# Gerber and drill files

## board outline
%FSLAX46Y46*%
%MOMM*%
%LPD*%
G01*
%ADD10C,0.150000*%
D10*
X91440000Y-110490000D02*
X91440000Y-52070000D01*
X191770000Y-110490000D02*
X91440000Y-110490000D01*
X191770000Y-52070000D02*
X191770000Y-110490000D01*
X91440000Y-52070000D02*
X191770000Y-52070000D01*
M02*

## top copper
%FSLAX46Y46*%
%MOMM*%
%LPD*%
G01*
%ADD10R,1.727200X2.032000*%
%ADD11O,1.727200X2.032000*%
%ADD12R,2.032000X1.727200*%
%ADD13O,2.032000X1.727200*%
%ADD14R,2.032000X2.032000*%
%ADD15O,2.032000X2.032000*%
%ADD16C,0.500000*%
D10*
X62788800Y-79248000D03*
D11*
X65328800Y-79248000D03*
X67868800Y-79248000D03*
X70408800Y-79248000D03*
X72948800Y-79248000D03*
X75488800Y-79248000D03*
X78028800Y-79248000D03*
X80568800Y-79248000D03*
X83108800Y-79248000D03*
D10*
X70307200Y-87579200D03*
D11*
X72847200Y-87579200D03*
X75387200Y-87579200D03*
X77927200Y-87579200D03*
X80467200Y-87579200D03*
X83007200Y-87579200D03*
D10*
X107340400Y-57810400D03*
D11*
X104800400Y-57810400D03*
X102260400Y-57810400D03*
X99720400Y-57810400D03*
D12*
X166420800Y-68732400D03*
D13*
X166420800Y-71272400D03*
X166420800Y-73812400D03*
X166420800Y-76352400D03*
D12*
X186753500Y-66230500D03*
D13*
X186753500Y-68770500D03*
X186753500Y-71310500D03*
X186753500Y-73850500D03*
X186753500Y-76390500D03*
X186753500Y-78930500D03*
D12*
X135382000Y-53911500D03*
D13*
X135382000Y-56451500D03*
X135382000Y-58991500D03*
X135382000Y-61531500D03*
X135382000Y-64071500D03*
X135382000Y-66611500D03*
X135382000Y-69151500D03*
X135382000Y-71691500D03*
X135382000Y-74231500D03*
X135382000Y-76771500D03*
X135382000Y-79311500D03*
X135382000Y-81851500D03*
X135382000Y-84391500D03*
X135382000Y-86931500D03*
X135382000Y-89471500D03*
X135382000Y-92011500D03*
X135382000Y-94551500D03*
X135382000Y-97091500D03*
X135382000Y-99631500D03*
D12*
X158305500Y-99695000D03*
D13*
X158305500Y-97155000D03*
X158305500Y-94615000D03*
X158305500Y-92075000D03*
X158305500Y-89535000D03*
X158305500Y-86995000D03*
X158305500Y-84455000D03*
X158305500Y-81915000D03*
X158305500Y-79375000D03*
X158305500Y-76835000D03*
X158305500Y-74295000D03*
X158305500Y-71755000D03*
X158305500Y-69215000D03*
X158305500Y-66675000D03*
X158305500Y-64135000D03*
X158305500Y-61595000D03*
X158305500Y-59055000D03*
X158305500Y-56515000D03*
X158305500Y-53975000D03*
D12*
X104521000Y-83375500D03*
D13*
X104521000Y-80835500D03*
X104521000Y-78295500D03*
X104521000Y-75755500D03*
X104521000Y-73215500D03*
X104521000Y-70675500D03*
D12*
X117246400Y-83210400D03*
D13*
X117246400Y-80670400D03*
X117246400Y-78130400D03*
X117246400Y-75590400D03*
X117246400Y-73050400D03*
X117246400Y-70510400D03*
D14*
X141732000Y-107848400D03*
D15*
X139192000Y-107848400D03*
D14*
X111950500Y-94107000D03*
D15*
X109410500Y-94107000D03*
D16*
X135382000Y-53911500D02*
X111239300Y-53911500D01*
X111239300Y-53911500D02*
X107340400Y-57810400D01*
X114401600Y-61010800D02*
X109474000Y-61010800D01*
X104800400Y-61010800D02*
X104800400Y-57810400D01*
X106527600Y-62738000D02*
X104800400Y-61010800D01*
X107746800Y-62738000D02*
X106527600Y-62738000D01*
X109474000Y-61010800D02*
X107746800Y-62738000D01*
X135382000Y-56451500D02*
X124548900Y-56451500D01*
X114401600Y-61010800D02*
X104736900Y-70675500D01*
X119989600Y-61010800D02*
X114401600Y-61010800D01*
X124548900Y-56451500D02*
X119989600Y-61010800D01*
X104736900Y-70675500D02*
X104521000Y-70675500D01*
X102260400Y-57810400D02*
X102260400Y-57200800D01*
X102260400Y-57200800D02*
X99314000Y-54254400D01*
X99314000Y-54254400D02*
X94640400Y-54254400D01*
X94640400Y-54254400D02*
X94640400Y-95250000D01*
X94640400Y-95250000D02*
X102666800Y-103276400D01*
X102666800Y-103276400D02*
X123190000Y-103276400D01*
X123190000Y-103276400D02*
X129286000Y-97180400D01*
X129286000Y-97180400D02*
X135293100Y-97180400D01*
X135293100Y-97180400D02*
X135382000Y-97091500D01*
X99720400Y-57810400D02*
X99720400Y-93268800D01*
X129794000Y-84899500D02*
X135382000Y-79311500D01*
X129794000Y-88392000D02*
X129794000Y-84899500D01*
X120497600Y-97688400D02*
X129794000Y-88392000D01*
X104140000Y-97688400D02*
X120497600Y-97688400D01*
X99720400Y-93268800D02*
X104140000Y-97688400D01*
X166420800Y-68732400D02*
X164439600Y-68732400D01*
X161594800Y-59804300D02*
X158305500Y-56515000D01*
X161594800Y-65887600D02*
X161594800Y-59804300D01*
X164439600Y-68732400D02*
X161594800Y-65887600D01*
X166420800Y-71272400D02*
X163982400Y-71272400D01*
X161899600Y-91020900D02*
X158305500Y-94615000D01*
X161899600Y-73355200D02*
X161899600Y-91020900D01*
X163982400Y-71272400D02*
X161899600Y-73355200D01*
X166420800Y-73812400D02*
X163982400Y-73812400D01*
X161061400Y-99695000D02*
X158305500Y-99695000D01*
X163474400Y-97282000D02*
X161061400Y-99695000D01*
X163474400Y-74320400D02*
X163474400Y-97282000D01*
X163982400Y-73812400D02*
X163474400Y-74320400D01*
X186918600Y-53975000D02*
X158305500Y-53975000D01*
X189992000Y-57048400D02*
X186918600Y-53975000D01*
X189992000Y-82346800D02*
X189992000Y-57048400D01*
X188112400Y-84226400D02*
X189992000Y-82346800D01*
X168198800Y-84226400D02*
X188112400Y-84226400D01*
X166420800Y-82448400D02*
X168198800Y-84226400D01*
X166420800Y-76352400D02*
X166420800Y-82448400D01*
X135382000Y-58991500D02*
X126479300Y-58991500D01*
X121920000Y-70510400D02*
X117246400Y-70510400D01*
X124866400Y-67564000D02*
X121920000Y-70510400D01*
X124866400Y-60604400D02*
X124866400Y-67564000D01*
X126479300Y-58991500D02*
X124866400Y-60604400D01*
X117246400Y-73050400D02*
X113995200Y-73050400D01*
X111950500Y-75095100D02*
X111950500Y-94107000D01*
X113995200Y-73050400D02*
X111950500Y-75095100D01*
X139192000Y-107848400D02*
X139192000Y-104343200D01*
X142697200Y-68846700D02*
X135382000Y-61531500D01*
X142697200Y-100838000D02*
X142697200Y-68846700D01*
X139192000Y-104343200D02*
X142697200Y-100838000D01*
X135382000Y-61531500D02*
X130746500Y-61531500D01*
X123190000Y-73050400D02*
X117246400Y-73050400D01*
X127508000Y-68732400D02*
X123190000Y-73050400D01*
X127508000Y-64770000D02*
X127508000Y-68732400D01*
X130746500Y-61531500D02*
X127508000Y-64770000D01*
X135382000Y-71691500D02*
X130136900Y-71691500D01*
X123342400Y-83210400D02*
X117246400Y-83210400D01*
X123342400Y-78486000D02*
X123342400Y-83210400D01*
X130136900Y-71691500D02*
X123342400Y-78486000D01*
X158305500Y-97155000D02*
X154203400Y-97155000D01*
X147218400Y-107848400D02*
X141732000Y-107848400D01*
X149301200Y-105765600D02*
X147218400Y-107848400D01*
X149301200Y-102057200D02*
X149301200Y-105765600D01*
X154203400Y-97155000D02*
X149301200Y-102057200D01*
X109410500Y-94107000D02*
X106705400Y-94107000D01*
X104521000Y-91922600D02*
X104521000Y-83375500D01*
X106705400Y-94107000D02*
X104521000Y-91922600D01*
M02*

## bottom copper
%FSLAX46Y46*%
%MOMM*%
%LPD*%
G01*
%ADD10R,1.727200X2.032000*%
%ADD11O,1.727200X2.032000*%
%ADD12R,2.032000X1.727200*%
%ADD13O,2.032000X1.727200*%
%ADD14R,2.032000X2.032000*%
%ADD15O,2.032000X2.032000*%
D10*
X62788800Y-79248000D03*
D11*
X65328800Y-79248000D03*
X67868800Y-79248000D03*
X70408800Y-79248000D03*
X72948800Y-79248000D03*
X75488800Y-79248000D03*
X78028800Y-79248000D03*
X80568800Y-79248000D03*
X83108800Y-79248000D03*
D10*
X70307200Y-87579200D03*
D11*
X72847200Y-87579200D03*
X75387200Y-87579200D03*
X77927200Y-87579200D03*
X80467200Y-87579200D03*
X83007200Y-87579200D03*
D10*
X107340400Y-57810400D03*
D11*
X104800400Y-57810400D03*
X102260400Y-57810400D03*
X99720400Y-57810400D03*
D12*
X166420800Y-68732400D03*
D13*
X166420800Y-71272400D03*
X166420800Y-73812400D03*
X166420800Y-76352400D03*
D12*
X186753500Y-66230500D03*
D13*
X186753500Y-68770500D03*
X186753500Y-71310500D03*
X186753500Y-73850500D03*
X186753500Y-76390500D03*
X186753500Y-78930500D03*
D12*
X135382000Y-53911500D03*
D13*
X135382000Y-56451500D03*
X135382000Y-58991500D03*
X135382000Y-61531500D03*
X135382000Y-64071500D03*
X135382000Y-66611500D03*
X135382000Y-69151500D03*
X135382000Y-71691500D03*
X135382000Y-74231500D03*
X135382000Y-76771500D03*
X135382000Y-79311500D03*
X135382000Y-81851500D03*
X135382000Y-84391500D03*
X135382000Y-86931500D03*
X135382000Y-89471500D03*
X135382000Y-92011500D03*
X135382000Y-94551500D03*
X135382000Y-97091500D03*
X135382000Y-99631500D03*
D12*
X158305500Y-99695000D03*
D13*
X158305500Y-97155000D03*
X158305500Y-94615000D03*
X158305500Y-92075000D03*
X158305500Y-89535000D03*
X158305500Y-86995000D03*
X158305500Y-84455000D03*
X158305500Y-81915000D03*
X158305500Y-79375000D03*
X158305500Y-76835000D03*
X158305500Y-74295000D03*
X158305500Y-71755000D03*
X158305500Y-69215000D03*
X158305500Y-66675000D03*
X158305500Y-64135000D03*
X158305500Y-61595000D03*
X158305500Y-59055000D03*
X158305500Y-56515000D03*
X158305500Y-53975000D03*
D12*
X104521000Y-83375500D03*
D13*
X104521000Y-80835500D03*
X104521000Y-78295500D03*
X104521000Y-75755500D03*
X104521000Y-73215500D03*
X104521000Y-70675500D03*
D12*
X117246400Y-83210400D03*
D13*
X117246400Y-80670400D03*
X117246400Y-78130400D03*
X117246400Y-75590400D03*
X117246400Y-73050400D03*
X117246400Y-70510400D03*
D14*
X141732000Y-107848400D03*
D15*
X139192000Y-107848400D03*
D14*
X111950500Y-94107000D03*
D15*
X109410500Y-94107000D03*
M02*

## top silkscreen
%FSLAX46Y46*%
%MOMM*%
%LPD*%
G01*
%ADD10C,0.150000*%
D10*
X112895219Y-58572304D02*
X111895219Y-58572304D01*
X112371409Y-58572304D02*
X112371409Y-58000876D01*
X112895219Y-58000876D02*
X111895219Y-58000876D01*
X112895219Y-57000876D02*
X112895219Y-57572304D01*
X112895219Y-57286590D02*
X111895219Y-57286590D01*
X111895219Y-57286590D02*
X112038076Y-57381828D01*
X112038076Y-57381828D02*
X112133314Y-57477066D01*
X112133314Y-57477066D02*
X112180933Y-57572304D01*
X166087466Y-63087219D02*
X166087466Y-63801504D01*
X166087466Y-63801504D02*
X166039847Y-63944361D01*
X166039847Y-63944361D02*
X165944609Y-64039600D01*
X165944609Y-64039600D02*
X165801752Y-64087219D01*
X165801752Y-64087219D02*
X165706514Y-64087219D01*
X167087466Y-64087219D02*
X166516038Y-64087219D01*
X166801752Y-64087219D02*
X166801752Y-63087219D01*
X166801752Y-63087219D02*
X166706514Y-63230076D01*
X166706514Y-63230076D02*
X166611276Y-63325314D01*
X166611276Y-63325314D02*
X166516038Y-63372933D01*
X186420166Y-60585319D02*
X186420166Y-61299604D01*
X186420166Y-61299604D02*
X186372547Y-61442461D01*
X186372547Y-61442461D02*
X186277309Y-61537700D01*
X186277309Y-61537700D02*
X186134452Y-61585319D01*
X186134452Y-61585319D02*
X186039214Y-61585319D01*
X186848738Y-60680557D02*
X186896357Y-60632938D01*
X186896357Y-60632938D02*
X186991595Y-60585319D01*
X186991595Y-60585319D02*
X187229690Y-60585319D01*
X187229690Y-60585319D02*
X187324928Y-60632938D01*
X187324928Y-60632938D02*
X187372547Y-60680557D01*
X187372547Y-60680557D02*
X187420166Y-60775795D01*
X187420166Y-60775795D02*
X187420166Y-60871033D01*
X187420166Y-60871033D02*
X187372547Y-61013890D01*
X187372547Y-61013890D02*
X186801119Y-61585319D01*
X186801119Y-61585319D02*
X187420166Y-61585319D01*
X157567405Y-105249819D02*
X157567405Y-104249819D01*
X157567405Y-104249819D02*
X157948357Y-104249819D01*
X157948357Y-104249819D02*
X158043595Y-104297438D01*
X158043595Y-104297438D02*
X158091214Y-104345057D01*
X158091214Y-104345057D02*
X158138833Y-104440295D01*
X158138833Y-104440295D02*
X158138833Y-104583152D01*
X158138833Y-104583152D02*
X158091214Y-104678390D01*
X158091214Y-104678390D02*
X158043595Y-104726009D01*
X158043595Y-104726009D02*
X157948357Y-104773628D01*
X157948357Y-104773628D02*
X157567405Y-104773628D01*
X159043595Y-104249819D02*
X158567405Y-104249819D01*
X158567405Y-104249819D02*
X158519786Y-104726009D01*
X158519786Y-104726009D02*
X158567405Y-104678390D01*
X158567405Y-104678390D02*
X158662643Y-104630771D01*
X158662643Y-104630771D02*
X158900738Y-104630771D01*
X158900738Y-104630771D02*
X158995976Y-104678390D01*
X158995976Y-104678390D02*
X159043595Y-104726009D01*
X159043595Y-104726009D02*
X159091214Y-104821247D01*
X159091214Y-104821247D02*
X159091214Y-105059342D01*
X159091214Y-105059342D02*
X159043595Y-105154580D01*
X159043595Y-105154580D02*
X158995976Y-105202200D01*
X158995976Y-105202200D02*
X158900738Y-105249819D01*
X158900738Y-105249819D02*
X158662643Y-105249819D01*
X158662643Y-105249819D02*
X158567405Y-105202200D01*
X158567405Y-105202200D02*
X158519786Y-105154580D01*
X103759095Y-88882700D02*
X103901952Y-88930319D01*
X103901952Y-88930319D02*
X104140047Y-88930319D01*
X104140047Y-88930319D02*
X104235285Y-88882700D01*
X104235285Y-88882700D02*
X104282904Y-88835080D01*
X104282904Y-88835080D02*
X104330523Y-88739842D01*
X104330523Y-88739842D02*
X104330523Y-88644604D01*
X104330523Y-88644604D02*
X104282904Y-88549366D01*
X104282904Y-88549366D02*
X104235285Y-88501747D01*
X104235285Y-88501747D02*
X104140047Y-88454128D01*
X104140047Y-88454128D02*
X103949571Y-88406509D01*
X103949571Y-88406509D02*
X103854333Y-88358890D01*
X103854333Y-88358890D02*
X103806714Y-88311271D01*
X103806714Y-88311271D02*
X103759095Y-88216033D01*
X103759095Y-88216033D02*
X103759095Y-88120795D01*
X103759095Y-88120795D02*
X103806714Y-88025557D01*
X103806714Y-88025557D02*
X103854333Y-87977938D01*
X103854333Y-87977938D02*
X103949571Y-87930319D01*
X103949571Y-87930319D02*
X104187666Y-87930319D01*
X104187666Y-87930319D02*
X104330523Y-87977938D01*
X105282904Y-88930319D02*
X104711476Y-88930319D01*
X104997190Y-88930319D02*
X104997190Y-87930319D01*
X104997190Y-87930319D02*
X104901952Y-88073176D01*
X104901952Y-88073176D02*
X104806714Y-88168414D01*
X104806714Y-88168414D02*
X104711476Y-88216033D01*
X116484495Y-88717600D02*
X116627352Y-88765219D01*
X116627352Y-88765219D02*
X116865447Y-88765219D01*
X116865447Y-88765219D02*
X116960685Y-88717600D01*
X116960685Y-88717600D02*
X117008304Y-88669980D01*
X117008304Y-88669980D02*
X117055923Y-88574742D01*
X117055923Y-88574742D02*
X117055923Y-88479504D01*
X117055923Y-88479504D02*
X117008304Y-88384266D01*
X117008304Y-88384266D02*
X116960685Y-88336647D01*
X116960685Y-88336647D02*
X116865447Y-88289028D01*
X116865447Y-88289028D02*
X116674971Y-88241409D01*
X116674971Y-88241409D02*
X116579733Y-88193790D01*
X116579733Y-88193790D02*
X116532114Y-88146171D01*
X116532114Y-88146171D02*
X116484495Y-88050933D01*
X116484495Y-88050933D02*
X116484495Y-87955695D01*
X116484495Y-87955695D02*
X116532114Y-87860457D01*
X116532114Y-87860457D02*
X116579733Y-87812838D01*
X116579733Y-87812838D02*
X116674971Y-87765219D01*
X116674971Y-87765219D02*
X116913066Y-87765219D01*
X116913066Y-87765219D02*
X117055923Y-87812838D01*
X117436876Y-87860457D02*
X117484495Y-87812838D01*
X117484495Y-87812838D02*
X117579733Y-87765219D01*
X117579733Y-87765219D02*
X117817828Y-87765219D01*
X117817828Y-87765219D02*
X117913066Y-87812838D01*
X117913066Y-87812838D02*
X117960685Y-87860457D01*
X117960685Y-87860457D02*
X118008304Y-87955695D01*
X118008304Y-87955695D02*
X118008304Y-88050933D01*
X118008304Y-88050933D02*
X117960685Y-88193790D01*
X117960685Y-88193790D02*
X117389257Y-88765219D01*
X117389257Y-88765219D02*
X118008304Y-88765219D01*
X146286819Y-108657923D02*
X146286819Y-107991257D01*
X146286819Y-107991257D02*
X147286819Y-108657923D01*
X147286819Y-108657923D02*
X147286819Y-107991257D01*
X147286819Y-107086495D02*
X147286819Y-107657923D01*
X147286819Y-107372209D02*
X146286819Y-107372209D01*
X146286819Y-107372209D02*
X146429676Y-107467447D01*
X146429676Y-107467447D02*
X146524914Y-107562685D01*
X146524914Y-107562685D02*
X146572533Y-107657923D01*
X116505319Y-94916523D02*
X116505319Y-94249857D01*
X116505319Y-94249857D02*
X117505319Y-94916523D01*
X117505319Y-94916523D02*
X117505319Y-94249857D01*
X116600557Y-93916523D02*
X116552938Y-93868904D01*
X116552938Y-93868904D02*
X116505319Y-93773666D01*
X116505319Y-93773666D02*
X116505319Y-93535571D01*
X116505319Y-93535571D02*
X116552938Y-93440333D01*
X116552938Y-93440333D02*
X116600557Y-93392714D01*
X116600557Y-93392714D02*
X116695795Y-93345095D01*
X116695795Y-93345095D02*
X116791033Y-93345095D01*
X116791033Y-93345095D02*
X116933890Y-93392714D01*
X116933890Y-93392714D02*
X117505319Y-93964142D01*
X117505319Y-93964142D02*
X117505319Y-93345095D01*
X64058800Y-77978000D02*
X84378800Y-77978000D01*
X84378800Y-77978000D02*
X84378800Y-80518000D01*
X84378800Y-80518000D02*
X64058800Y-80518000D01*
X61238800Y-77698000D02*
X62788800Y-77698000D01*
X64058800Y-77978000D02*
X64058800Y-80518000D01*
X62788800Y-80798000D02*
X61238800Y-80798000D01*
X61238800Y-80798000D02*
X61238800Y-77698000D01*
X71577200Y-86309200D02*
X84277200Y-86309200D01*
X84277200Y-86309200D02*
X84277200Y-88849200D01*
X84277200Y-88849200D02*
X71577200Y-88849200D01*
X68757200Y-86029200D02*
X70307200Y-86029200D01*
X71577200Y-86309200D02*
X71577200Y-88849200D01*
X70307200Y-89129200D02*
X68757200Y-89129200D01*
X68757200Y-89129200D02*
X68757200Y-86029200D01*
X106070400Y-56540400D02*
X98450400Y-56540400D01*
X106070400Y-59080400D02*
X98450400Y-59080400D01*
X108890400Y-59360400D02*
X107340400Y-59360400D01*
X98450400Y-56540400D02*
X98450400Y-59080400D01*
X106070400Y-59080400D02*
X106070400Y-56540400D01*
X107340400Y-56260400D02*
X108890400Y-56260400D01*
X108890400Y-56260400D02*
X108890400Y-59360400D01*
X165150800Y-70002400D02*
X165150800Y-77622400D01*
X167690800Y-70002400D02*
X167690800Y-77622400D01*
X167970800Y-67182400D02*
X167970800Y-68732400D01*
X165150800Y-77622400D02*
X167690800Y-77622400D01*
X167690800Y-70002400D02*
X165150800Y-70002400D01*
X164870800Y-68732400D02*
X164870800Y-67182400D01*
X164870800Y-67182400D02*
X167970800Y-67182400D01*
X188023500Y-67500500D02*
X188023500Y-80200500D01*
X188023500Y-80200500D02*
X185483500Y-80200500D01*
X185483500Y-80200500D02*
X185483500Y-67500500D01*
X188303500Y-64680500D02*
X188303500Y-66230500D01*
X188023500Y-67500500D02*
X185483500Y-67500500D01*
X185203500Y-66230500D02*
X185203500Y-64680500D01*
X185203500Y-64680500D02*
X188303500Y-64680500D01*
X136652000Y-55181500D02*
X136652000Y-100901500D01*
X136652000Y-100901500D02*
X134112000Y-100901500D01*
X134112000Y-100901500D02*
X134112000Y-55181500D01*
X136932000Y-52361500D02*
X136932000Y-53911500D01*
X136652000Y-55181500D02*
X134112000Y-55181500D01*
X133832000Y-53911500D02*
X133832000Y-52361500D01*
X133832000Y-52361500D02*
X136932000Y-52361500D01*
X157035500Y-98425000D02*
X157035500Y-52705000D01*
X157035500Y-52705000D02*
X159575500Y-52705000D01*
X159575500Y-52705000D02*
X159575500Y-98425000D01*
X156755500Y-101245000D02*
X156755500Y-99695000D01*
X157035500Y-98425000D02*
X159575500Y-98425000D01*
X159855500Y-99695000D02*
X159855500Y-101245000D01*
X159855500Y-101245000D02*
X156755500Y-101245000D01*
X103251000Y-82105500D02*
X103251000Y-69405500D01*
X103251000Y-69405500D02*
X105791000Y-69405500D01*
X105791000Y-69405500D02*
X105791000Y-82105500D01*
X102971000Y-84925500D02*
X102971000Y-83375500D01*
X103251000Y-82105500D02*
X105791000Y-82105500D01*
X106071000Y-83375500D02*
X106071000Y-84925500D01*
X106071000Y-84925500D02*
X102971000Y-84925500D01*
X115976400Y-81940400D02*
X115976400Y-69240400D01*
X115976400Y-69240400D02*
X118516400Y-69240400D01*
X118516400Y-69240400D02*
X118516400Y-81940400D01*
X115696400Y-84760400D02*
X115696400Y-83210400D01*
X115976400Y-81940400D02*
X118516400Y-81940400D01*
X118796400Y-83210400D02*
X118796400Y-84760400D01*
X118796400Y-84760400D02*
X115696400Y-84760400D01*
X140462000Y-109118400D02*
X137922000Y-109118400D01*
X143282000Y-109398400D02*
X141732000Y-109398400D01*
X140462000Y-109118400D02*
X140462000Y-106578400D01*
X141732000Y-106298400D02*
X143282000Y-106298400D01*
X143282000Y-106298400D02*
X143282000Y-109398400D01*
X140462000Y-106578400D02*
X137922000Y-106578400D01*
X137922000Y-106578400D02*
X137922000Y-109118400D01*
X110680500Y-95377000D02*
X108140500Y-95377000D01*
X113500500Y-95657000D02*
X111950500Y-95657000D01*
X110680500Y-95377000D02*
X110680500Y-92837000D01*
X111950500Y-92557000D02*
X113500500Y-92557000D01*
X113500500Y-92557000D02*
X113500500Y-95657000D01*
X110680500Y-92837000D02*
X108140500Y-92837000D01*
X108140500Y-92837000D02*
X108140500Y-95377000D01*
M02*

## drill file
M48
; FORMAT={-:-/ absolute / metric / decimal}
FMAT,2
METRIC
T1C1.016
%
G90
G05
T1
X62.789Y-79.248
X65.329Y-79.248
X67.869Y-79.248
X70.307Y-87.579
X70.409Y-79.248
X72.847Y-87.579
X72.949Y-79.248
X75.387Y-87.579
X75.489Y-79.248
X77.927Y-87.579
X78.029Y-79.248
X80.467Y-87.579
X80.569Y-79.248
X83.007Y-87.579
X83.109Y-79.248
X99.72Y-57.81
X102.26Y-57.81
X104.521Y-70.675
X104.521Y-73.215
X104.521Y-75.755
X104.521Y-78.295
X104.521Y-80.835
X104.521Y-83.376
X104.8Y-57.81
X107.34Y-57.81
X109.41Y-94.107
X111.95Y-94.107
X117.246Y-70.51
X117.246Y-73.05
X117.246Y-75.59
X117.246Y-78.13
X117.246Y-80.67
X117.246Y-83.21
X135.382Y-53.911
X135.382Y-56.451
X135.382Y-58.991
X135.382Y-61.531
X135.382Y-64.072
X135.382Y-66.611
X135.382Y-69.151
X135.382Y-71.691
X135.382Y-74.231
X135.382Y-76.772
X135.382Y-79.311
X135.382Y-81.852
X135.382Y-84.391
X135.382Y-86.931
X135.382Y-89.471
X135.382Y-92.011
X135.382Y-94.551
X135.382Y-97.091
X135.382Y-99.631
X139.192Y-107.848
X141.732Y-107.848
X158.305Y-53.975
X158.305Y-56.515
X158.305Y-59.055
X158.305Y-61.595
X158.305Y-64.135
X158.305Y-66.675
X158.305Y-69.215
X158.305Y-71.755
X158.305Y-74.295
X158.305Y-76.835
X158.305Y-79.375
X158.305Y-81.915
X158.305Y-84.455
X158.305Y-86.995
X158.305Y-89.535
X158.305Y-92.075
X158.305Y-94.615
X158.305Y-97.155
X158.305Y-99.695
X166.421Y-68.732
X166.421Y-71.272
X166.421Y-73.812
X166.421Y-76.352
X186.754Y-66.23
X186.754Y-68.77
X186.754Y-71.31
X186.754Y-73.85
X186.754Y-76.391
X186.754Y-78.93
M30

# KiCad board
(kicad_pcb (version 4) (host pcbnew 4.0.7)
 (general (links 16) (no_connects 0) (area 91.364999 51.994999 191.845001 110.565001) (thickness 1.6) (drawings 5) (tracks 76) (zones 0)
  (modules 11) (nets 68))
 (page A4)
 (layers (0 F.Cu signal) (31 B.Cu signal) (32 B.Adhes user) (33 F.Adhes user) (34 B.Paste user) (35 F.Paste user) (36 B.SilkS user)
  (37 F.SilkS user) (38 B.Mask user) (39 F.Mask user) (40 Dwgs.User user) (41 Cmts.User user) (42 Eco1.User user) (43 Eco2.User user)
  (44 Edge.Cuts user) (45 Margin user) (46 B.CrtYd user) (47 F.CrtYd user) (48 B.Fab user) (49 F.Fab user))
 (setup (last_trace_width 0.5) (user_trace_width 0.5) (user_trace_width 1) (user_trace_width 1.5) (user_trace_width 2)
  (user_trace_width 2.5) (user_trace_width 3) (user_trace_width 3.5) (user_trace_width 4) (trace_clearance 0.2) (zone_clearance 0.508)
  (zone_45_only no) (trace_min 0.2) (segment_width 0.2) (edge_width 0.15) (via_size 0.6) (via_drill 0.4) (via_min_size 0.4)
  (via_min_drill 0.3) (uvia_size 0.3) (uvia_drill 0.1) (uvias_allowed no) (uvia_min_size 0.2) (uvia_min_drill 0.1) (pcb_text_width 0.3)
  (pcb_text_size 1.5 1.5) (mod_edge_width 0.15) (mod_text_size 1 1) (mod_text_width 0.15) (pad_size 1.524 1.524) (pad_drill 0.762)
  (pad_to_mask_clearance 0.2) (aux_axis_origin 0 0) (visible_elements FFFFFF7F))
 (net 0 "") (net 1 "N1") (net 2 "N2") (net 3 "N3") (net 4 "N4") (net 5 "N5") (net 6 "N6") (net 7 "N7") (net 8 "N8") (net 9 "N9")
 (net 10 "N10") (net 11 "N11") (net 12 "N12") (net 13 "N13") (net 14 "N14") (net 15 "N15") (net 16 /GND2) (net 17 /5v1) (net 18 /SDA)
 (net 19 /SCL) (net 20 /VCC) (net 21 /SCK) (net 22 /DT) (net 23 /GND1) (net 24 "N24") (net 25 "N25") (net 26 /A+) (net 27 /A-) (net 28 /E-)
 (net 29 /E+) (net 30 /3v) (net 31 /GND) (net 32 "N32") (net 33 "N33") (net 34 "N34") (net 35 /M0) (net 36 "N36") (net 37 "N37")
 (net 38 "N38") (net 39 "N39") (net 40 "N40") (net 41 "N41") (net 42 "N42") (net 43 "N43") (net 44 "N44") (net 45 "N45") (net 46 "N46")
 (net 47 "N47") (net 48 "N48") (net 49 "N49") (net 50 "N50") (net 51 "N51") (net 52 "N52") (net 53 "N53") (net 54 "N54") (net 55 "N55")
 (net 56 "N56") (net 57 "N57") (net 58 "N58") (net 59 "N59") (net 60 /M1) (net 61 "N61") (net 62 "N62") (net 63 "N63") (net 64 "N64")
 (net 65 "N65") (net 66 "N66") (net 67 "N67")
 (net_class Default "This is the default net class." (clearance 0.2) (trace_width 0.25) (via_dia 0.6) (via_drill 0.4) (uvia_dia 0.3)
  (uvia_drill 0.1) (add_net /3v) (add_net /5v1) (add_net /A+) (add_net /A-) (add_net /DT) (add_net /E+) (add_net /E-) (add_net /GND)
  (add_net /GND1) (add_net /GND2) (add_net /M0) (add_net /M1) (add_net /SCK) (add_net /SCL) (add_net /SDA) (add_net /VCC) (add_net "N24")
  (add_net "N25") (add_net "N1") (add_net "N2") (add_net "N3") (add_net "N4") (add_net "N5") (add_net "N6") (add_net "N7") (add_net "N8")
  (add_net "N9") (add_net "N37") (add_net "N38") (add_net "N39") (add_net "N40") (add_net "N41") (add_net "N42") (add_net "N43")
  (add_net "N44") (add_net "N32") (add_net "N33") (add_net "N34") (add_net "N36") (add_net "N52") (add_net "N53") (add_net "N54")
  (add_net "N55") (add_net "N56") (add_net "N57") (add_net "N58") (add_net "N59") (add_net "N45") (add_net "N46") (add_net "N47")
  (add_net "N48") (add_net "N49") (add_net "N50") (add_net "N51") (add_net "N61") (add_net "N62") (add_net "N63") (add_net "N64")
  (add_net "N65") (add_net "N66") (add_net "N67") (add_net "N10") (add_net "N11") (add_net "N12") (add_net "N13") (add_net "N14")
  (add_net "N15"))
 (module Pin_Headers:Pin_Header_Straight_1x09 (layer F.Cu) (at 62.7888 79.248 90)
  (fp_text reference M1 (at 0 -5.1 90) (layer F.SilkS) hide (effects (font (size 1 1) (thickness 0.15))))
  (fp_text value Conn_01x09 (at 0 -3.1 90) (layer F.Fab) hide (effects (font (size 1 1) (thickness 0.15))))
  (fp_line (start 1.27 1.27) (end 1.27 21.59) (layer F.SilkS) (width 0.15))
  (fp_line (start 1.27 21.59) (end -1.27 21.59) (layer F.SilkS) (width 0.15))
  (fp_line (start -1.27 21.59) (end -1.27 1.27) (layer F.SilkS) (width 0.15))
  (fp_line (start 1.55 -1.55) (end 1.55 0) (layer F.SilkS) (width 0.15))
  (fp_line (start 1.27 1.27) (end -1.27 1.27) (layer F.SilkS) (width 0.15))
  (fp_line (start -1.55 0) (end -1.55 -1.55) (layer F.SilkS) (width 0.15))
  (fp_line (start -1.55 -1.55) (end 1.55 -1.55) (layer F.SilkS) (width 0.15))
  (pad 1 thru_hole rect (at 0 0 90) (size 2.032 1.7272) (drill 1.016) (layers *.Cu *.Mask) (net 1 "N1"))
  (pad 2 thru_hole oval (at 0 2.54 90) (size 2.032 1.7272) (drill 1.016) (layers *.Cu *.Mask) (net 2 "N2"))
  (pad 3 thru_hole oval (at 0 5.08 90) (size 2.032 1.7272) (drill 1.016) (layers *.Cu *.Mask) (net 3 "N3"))
  (pad 4 thru_hole oval (at 0 7.62 90) (size 2.032 1.7272) (drill 1.016) (layers *.Cu *.Mask) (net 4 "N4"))
  (pad 5 thru_hole oval (at 0 10.16 90) (size 2.032 1.7272) (drill 1.016) (layers *.Cu *.Mask) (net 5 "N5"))
  (pad 6 thru_hole oval (at 0 12.7 90) (size 2.032 1.7272) (drill 1.016) (layers *.Cu *.Mask) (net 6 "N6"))
  (pad 7 thru_hole oval (at 0 15.24 90) (size 2.032 1.7272) (drill 1.016) (layers *.Cu *.Mask) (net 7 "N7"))
  (pad 8 thru_hole oval (at 0 17.78 90) (size 2.032 1.7272) (drill 1.016) (layers *.Cu *.Mask) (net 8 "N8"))
  (pad 9 thru_hole oval (at 0 20.32 90) (size 2.032 1.7272) (drill 1.016) (layers *.Cu *.Mask) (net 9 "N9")))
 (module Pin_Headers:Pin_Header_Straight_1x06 (layer F.Cu) (at 70.3072 87.5792 90)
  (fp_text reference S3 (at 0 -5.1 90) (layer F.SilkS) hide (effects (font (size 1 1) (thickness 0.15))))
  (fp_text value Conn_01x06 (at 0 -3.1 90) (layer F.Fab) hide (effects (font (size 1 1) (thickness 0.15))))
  (fp_line (start 1.27 1.27) (end 1.27 13.97) (layer F.SilkS) (width 0.15))
  (fp_line (start 1.27 13.97) (end -1.27 13.97) (layer F.SilkS) (width 0.15))
  (fp_line (start -1.27 13.97) (end -1.27 1.27) (layer F.SilkS) (width 0.15))
  (fp_line (start 1.55 -1.55) (end 1.55 0) (layer F.SilkS) (width 0.15))
  (fp_line (start 1.27 1.27) (end -1.27 1.27) (layer F.SilkS) (width 0.15))
  (fp_line (start -1.55 0) (end -1.55 -1.55) (layer F.SilkS) (width 0.15))
  (fp_line (start -1.55 -1.55) (end 1.55 -1.55) (layer F.SilkS) (width 0.15))
  (pad 1 thru_hole rect (at 0 0 90) (size 2.032 1.7272) (drill 1.016) (layers *.Cu *.Mask) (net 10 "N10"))
  (pad 2 thru_hole oval (at 0 2.54 90) (size 2.032 1.7272) (drill 1.016) (layers *.Cu *.Mask) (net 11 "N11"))
  (pad 3 thru_hole oval (at 0 5.08 90) (size 2.032 1.7272) (drill 1.016) (layers *.Cu *.Mask) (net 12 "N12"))
  (pad 4 thru_hole oval (at 0 7.62 90) (size 2.032 1.7272) (drill 1.016) (layers *.Cu *.Mask) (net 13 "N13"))
  (pad 5 thru_hole oval (at 0 10.16 90) (size 2.032 1.7272) (drill 1.016) (layers *.Cu *.Mask) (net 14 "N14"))
  (pad 6 thru_hole oval (at 0 12.7 90) (size 2.032 1.7272) (drill 1.016) (layers *.Cu *.Mask) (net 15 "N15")))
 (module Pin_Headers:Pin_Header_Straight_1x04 (layer F.Cu) (at 107.3404 57.8104 270)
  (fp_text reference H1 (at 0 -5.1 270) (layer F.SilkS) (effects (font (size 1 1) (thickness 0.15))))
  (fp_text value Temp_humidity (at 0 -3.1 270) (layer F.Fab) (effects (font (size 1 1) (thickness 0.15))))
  (fp_line (start -1.27 1.27) (end -1.27 8.89) (layer F.SilkS) (width 0.15))
  (fp_line (start 1.27 1.27) (end 1.27 8.89) (layer F.SilkS) (width 0.15))
  (fp_line (start 1.55 -1.55) (end 1.55 0) (layer F.SilkS) (width 0.15))
  (fp_line (start -1.27 8.89) (end 1.27 8.89) (layer F.SilkS) (width 0.15))
  (fp_line (start 1.27 1.27) (end -1.27 1.27) (layer F.SilkS) (width 0.15))
  (fp_line (start -1.55 0) (end -1.55 -1.55) (layer F.SilkS) (width 0.15))
  (fp_line (start -1.55 -1.55) (end 1.55 -1.55) (layer F.SilkS) (width 0.15))
  (pad 1 thru_hole rect (at 0 0 270) (size 2.032 1.7272) (drill 1.016) (layers *.Cu *.Mask) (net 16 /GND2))
  (pad 2 thru_hole oval (at 0 2.54 270) (size 2.032 1.7272) (drill 1.016) (layers *.Cu *.Mask) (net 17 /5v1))
  (pad 3 thru_hole oval (at 0 5.08 270) (size 2.032 1.7272) (drill 1.016) (layers *.Cu *.Mask) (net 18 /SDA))
  (pad 4 thru_hole oval (at 0 7.62 270) (size 2.032 1.7272) (drill 1.016) (layers *.Cu *.Mask) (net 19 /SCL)))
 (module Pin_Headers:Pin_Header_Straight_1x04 (layer F.Cu) (at 166.4208 68.7324)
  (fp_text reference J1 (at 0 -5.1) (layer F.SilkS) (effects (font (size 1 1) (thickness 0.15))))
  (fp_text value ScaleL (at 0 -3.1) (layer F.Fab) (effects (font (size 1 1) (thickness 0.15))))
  (fp_line (start -1.27 1.27) (end -1.27 8.89) (layer F.SilkS) (width 0.15))
  (fp_line (start 1.27 1.27) (end 1.27 8.89) (layer F.SilkS) (width 0.15))
  (fp_line (start 1.55 -1.55) (end 1.55 0) (layer F.SilkS) (width 0.15))
  (fp_line (start -1.27 8.89) (end 1.27 8.89) (layer F.SilkS) (width 0.15))
  (fp_line (start 1.27 1.27) (end -1.27 1.27) (layer F.SilkS) (width 0.15))
  (fp_line (start -1.55 0) (end -1.55 -1.55) (layer F.SilkS) (width 0.15))
  (fp_line (start -1.55 -1.55) (end 1.55 -1.55) (layer F.SilkS) (width 0.15))
  (pad 1 thru_hole rect (at 0 0) (size 2.032 1.7272) (drill 1.016) (layers *.Cu *.Mask) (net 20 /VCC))
  (pad 2 thru_hole oval (at 0 2.54) (size 2.032 1.7272) (drill 1.016) (layers *.Cu *.Mask) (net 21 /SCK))
  (pad 3 thru_hole oval (at 0 5.08) (size 2.032 1.7272) (drill 1.016) (layers *.Cu *.Mask) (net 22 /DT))
  (pad 4 thru_hole oval (at 0 7.62) (size 2.032 1.7272) (drill 1.016) (layers *.Cu *.Mask) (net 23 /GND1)))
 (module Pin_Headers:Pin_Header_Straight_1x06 (layer F.Cu) (at 186.7535 66.2305)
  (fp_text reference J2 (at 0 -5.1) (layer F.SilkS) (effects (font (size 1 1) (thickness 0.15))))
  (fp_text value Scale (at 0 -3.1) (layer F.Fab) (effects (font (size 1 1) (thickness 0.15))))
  (fp_line (start 1.27 1.27) (end 1.27 13.97) (layer F.SilkS) (width 0.15))
  (fp_line (start 1.27 13.97) (end -1.27 13.97) (layer F.SilkS) (width 0.15))
  (fp_line (start -1.27 13.97) (end -1.27 1.27) (layer F.SilkS) (width 0.15))
  (fp_line (start 1.55 -1.55) (end 1.55 0) (layer F.SilkS) (width 0.15))
  (fp_line (start 1.27 1.27) (end -1.27 1.27) (layer F.SilkS) (width 0.15))
  (fp_line (start -1.55 0) (end -1.55 -1.55) (layer F.SilkS) (width 0.15))
  (fp_line (start -1.55 -1.55) (end 1.55 -1.55) (layer F.SilkS) (width 0.15))
  (pad 1 thru_hole rect (at 0 0) (size 2.032 1.7272) (drill 1.016) (layers *.Cu *.Mask) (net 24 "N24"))
  (pad 2 thru_hole oval (at 0 2.54) (size 2.032 1.7272) (drill 1.016) (layers *.Cu *.Mask) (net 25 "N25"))
  (pad 3 thru_hole oval (at 0 5.08) (size 2.032 1.7272) (drill 1.016) (layers *.Cu *.Mask) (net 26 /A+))
  (pad 4 thru_hole oval (at 0 7.62) (size 2.032 1.7272) (drill 1.016) (layers *.Cu *.Mask) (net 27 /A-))
  (pad 5 thru_hole oval (at 0 10.16) (size 2.032 1.7272) (drill 1.016) (layers *.Cu *.Mask) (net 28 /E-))
  (pad 6 thru_hole oval (at 0 12.7) (size 2.032 1.7272) (drill 1.016) (layers *.Cu *.Mask) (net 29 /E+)))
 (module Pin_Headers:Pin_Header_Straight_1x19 (layer F.Cu) (at 135.382 53.9115)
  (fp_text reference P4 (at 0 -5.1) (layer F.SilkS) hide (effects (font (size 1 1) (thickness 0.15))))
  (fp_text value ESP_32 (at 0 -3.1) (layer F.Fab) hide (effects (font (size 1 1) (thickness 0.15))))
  (fp_line (start 1.27 1.27) (end 1.27 46.99) (layer F.SilkS) (width 0.15))
  (fp_line (start 1.27 46.99) (end -1.27 46.99) (layer F.SilkS) (width 0.15))
  (fp_line (start -1.27 46.99) (end -1.27 1.27) (layer F.SilkS) (width 0.15))
  (fp_line (start 1.55 -1.55) (end 1.55 0) (layer F.SilkS) (width 0.15))
  (fp_line (start 1.27 1.27) (end -1.27 1.27) (layer F.SilkS) (width 0.15))
  (fp_line (start -1.55 0) (end -1.55 -1.55) (layer F.SilkS) (width 0.15))
  (fp_line (start -1.55 -1.55) (end 1.55 -1.55) (layer F.SilkS) (width 0.15))
  (pad 1 thru_hole rect (at 0 0) (size 2.032 1.7272) (drill 1.016) (layers *.Cu *.Mask) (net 16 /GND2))
  (pad 2 thru_hole oval (at 0 2.54) (size 2.032 1.7272) (drill 1.016) (layers *.Cu *.Mask) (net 17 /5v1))
  (pad 3 thru_hole oval (at 0 5.08) (size 2.032 1.7272) (drill 1.016) (layers *.Cu *.Mask) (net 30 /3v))
  (pad 4 thru_hole oval (at 0 7.62) (size 2.032 1.7272) (drill 1.016) (layers *.Cu *.Mask) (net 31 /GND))
  (pad 5 thru_hole oval (at 0 10.16) (size 2.032 1.7272) (drill 1.016) (layers *.Cu *.Mask) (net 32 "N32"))
  (pad 6 thru_hole oval (at 0 12.7) (size 2.032 1.7272) (drill 1.016) (layers *.Cu *.Mask) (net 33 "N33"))
  (pad 7 thru_hole oval (at 0 15.24) (size 2.032 1.7272) (drill 1.016) (layers *.Cu *.Mask) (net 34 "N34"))
  (pad 8 thru_hole oval (at 0 17.78) (size 2.032 1.7272) (drill 1.016) (layers *.Cu *.Mask) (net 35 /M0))
  (pad 9 thru_hole oval (at 0 20.32) (size 2.032 1.7272) (drill 1.016) (layers *.Cu *.Mask) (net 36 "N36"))
  (pad 10 thru_hole oval (at 0 22.86) (size 2.032 1.7272) (drill 1.016) (layers *.Cu *.Mask) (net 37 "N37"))
  (pad 11 thru_hole oval (at 0 25.4) (size 2.032 1.7272) (drill 1.016) (layers *.Cu *.Mask) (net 19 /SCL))
  (pad 12 thru_hole oval (at 0 27.94) (size 2.032 1.7272) (drill 1.016) (layers *.Cu *.Mask) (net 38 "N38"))
  (pad 13 thru_hole oval (at 0 30.48) (size 2.032 1.7272) (drill 1.016) (layers *.Cu *.Mask) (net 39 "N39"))
  (pad 14 thru_hole oval (at 0 33.02) (size 2.032 1.7272) (drill 1.016) (layers *.Cu *.Mask) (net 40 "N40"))
  (pad 15 thru_hole oval (at 0 35.56) (size 2.032 1.7272) (drill 1.016) (layers *.Cu *.Mask) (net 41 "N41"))
  (pad 16 thru_hole oval (at 0 38.1) (size 2.032 1.7272) (drill 1.016) (layers *.Cu *.Mask) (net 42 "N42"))
  (pad 17 thru_hole oval (at 0 40.64) (size 2.032 1.7272) (drill 1.016) (layers *.Cu *.Mask) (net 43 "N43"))
  (pad 18 thru_hole oval (at 0 43.18) (size 2.032 1.7272) (drill 1.016) (layers *.Cu *.Mask) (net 18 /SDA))
  (pad 19 thru_hole oval (at 0 45.72) (size 2.032 1.7272) (drill 1.016) (layers *.Cu *.Mask) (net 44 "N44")))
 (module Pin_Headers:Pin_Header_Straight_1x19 (layer F.Cu) (at 158.3055 99.695 180)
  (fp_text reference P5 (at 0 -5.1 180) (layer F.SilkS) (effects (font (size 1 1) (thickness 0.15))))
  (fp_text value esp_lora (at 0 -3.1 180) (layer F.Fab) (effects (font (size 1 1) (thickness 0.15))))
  (fp_line (start 1.27 1.27) (end 1.27 46.99) (layer F.SilkS) (width 0.15))
  (fp_line (start 1.27 46.99) (end -1.27 46.99) (layer F.SilkS) (width 0.15))
  (fp_line (start -1.27 46.99) (end -1.27 1.27) (layer F.SilkS) (width 0.15))
  (fp_line (start 1.55 -1.55) (end 1.55 0) (layer F.SilkS) (width 0.15))
  (fp_line (start 1.27 1.27) (end -1.27 1.27) (layer F.SilkS) (width 0.15))
  (fp_line (start -1.55 0) (end -1.55 -1.55) (layer F.SilkS) (width 0.15))
  (fp_line (start -1.55 -1.55) (end 1.55 -1.55) (layer F.SilkS) (width 0.15))
  (pad 1 thru_hole rect (at 0 0 180) (size 2.032 1.7272) (drill 1.016) (layers *.Cu *.Mask) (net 22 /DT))
  (pad 2 thru_hole oval (at 0 2.54 180) (size 2.032 1.7272) (drill 1.016) (layers *.Cu *.Mask) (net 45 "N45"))
  (pad 3 thru_hole oval (at 0 5.08 180) (size 2.032 1.7272) (drill 1.016) (layers *.Cu *.Mask) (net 21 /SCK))
  (pad 4 thru_hole oval (at 0 7.62 180) (size 2.032 1.7272) (drill 1.016) (layers *.Cu *.Mask) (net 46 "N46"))
  (pad 5 thru_hole oval (at 0 10.16 180) (size 2.032 1.7272) (drill 1.016) (layers *.Cu *.Mask) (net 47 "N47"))
  (pad 6 thru_hole oval (at 0 12.7 180) (size 2.032 1.7272) (drill 1.016) (layers *.Cu *.Mask) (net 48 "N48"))
  (pad 7 thru_hole oval (at 0 15.24 180) (size 2.032 1.7272) (drill 1.016) (layers *.Cu *.Mask) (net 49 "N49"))
  (pad 8 thru_hole oval (at 0 17.78 180) (size 2.032 1.7272) (drill 1.016) (layers *.Cu *.Mask) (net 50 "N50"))
  (pad 9 thru_hole oval (at 0 20.32 180) (size 2.032 1.7272) (drill 1.016) (layers *.Cu *.Mask) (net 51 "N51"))
  (pad 10 thru_hole oval (at 0 22.86 180) (size 2.032 1.7272) (drill 1.016) (layers *.Cu *.Mask) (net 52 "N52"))
  (pad 11 thru_hole oval (at 0 25.4 180) (size 2.032 1.7272) (drill 1.016) (layers *.Cu *.Mask) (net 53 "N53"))
  (pad 12 thru_hole oval (at 0 27.94 180) (size 2.032 1.7272) (drill 1.016) (layers *.Cu *.Mask) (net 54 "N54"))
  (pad 13 thru_hole oval (at 0 30.48 180) (size 2.032 1.7272) (drill 1.016) (layers *.Cu *.Mask) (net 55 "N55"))
  (pad 14 thru_hole oval (at 0 33.02 180) (size 2.032 1.7272) (drill 1.016) (layers *.Cu *.Mask) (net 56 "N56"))
  (pad 15 thru_hole oval (at 0 35.56 180) (size 2.032 1.7272) (drill 1.016) (layers *.Cu *.Mask) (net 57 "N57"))
  (pad 16 thru_hole oval (at 0 38.1 180) (size 2.032 1.7272) (drill 1.016) (layers *.Cu *.Mask) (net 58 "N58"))
  (pad 17 thru_hole oval (at 0 40.64 180) (size 2.032 1.7272) (drill 1.016) (layers *.Cu *.Mask) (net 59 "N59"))
  (pad 18 thru_hole oval (at 0 43.18 180) (size 2.032 1.7272) (drill 1.016) (layers *.Cu *.Mask) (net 20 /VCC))
  (pad 19 thru_hole oval (at 0 45.72 180) (size 2.032 1.7272) (drill 1.016) (layers *.Cu *.Mask) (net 23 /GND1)))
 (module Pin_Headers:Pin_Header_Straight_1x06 (layer F.Cu) (at 104.521 83.3755 180)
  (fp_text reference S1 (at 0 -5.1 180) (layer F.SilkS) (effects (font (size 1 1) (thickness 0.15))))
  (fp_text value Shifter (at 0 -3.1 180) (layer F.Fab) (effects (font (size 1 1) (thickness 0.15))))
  (fp_line (start 1.27 1.27) (end 1.27 13.97) (layer F.SilkS) (width 0.15))
  (fp_line (start 1.27 13.97) (end -1.27 13.97) (layer F.SilkS) (width 0.15))
  (fp_line (start -1.27 13.97) (end -1.27 1.27) (layer F.SilkS) (width 0.15))
  (fp_line (start 1.55 -1.55) (end 1.55 0) (layer F.SilkS) (width 0.15))
  (fp_line (start 1.27 1.27) (end -1.27 1.27) (layer F.SilkS) (width 0.15))
  (fp_line (start -1.55 0) (end -1.55 -1.55) (layer F.SilkS) (width 0.15))
  (fp_line (start -1.55 -1.55) (end 1.55 -1.55) (layer F.SilkS) (width 0.15))
  (pad 1 thru_hole rect (at 0 0 180) (size 2.032 1.7272) (drill 1.016) (layers *.Cu *.Mask) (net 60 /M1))
  (pad 2 thru_hole oval (at 0 2.54 180) (size 2.032 1.7272) (drill 1.016) (layers *.Cu *.Mask) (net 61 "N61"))
  (pad 3 thru_hole oval (at 0 5.08 180) (size 2.032 1.7272) (drill 1.016) (layers *.Cu *.Mask) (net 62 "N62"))
  (pad 4 thru_hole oval (at 0 7.62 180) (size 2.032 1.7272) (drill 1.016) (layers *.Cu *.Mask) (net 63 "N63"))
  (pad 5 thru_hole oval (at 0 10.16 180) (size 2.032 1.7272) (drill 1.016) (layers *.Cu *.Mask) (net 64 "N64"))
  (pad 6 thru_hole oval (at 0 12.7 180) (size 2.032 1.7272) (drill 1.016) (layers *.Cu *.Mask) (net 17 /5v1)))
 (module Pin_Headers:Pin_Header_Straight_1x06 (layer F.Cu) (at 117.2464 83.2104 180)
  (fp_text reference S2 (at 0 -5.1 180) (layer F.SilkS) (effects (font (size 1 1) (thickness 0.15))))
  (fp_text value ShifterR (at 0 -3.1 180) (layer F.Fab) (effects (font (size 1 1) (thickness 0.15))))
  (fp_line (start 1.27 1.27) (end 1.27 13.97) (layer F.SilkS) (width 0.15))
  (fp_line (start 1.27 13.97) (end -1.27 13.97) (layer F.SilkS) (width 0.15))
  (fp_line (start -1.27 13.97) (end -1.27 1.27) (layer F.SilkS) (width 0.15))
  (fp_line (start 1.55 -1.55) (end 1.55 0) (layer F.SilkS) (width 0.15))
  (fp_line (start 1.27 1.27) (end -1.27 1.27) (layer F.SilkS) (width 0.15))
  (fp_line (start -1.55 0) (end -1.55 -1.55) (layer F.SilkS) (width 0.15))
  (fp_line (start -1.55 -1.55) (end 1.55 -1.55) (layer F.SilkS) (width 0.15))
  (pad 1 thru_hole rect (at 0 0 180) (size 2.032 1.7272) (drill 1.016) (layers *.Cu *.Mask) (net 35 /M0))
  (pad 2 thru_hole oval (at 0 2.54 180) (size 2.032 1.7272) (drill 1.016) (layers *.Cu *.Mask) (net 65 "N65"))
  (pad 3 thru_hole oval (at 0 5.08 180) (size 2.032 1.7272) (drill 1.016) (layers *.Cu *.Mask) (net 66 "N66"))
  (pad 4 thru_hole oval (at 0 7.62 180) (size 2.032 1.7272) (drill 1.016) (layers *.Cu *.Mask) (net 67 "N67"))
  (pad 5 thru_hole oval (at 0 10.16 180) (size 2.032 1.7272) (drill 1.016) (layers *.Cu *.Mask) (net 31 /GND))
  (pad 6 thru_hole oval (at 0 12.7 180) (size 2.032 1.7272) (drill 1.016) (layers *.Cu *.Mask) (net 30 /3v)))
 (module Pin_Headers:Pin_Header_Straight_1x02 (layer F.Cu) (at 141.732 107.8484 270)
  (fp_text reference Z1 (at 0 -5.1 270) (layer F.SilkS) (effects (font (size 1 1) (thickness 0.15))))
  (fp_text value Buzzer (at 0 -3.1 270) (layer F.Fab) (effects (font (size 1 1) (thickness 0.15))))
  (fp_line (start 1.27 1.27) (end 1.27 3.81) (layer F.SilkS) (width 0.15))
  (fp_line (start 1.55 -1.55) (end 1.55 0) (layer F.SilkS) (width 0.15))
  (fp_line (start 1.27 1.27) (end -1.27 1.27) (layer F.SilkS) (width 0.15))
  (fp_line (start -1.55 0) (end -1.55 -1.55) (layer F.SilkS) (width 0.15))
  (fp_line (start -1.55 -1.55) (end 1.55 -1.55) (layer F.SilkS) (width 0.15))
  (fp_line (start -1.27 1.27) (end -1.27 3.81) (layer F.SilkS) (width 0.15))
  (fp_line (start -1.27 3.81) (end 1.27 3.81) (layer F.SilkS) (width 0.15))
  (pad 1 thru_hole rect (at 0 0 270) (size 2.032 2.032) (drill 1.016) (layers *.Cu *.Mask) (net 45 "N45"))
  (pad 2 thru_hole oval (at 0 2.54 270) (size 2.032 2.032) (drill 1.016) (layers *.Cu *.Mask) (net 31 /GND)))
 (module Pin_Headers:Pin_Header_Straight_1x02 (layer F.Cu) (at 111.9505 94.107 270)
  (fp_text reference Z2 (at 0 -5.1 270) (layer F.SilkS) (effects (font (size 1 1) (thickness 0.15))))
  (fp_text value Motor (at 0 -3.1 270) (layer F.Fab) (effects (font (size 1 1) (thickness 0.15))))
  (fp_line (start 1.27 1.27) (end 1.27 3.81) (layer F.SilkS) (width 0.15))
  (fp_line (start 1.55 -1.55) (end 1.55 0) (layer F.SilkS) (width 0.15))
  (fp_line (start 1.27 1.27) (end -1.27 1.27) (layer F.SilkS) (width 0.15))
  (fp_line (start -1.55 0) (end -1.55 -1.55) (layer F.SilkS) (width 0.15))
  (fp_line (start -1.55 -1.55) (end 1.55 -1.55) (layer F.SilkS) (width 0.15))
  (fp_line (start -1.27 1.27) (end -1.27 3.81) (layer F.SilkS) (width 0.15))
  (fp_line (start -1.27 3.81) (end 1.27 3.81) (layer F.SilkS) (width 0.15))
  (pad 1 thru_hole rect (at 0 0 270) (size 2.032 2.032) (drill 1.016) (layers *.Cu *.Mask) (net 31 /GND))
  (pad 2 thru_hole oval (at 0 2.54 270) (size 2.032 2.032) (drill 1.016) (layers *.Cu *.Mask) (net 60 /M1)))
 (gr_line (start 91.44 110.49) (end 91.44 52.07) (angle 90) (layer Edge.Cuts) (width 0.15))
 (gr_line (start 191.77 110.49) (end 91.44 110.49) (angle 90) (layer Edge.Cuts) (width 0.15))
 (gr_line (start 191.77 52.07) (end 191.77 110.49) (angle 90) (layer Edge.Cuts) (width 0.15))
 (gr_line (start 91.44 52.07) (end 191.77 52.07) (angle 90) (layer Edge.Cuts) (width 0.15))
 (segment (start 135.382 53.9115) (end 111.2393 53.9115) (width 0.5) (layer F.Cu) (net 16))
 (segment (start 111.2393 53.9115) (end 107.3404 57.8104) (width 0.5) (layer F.Cu) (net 16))
 (segment (start 114.4016 61.0108) (end 109.474 61.0108) (width 0.5) (layer F.Cu) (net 17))
 (segment (start 104.8004 61.0108) (end 104.8004 57.8104) (width 0.5) (layer F.Cu) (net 17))
 (segment (start 106.5276 62.738) (end 104.8004 61.0108) (width 0.5) (layer F.Cu) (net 17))
 (segment (start 107.7468 62.738) (end 106.5276 62.738) (width 0.5) (layer F.Cu) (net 17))
 (segment (start 109.474 61.0108) (end 107.7468 62.738) (width 0.5) (layer F.Cu) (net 17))
 (segment (start 135.382 56.4515) (end 124.5489 56.4515) (width 0.5) (layer F.Cu) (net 17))
 (segment (start 114.4016 61.0108) (end 104.7369 70.6755) (width 0.5) (layer F.Cu) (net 17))
 (segment (start 119.9896 61.0108) (end 114.4016 61.0108) (width 0.5) (layer F.Cu) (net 17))
 (segment (start 124.5489 56.4515) (end 119.9896 61.0108) (width 0.5) (layer F.Cu) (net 17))
 (segment (start 104.7369 70.6755) (end 104.521 70.6755) (width 0.5) (layer F.Cu) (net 17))
 (segment (start 102.2604 57.8104) (end 102.2604 57.2008) (width 0.5) (layer F.Cu) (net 18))
 (segment (start 102.2604 57.2008) (end 99.314 54.2544) (width 0.5) (layer F.Cu) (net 18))
 (segment (start 99.314 54.2544) (end 94.6404 54.2544) (width 0.5) (layer F.Cu) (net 18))
 (segment (start 94.6404 54.2544) (end 94.6404 95.25) (width 0.5) (layer F.Cu) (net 18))
 (segment (start 94.6404 95.25) (end 102.6668 103.2764) (width 0.5) (layer F.Cu) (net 18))
 (segment (start 102.6668 103.2764) (end 123.19 103.2764) (width 0.5) (layer F.Cu) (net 18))
 (segment (start 123.19 103.2764) (end 129.286 97.1804) (width 0.5) (layer F.Cu) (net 18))
 (segment (start 129.286 97.1804) (end 135.2931 97.1804) (width 0.5) (layer F.Cu) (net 18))
 (segment (start 135.2931 97.1804) (end 135.382 97.0915) (width 0.5) (layer F.Cu) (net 18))
 (segment (start 99.7204 57.8104) (end 99.7204 93.2688) (width 0.5) (layer F.Cu) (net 19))
 (segment (start 129.794 84.8995) (end 135.382 79.3115) (width 0.5) (layer F.Cu) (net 19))
 (segment (start 129.794 88.392) (end 129.794 84.8995) (width 0.5) (layer F.Cu) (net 19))
 (segment (start 120.4976 97.6884) (end 129.794 88.392) (width 0.5) (layer F.Cu) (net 19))
 (segment (start 104.14 97.6884) (end 120.4976 97.6884) (width 0.5) (layer F.Cu) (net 19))
 (segment (start 99.7204 93.2688) (end 104.14 97.6884) (width 0.5) (layer F.Cu) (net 19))
 (segment (start 166.4208 68.7324) (end 164.4396 68.7324) (width 0.5) (layer F.Cu) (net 20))
 (segment (start 161.5948 59.8043) (end 158.3055 56.515) (width 0.5) (layer F.Cu) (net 20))
 (segment (start 161.5948 65.8876) (end 161.5948 59.8043) (width 0.5) (layer F.Cu) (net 20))
 (segment (start 164.4396 68.7324) (end 161.5948 65.8876) (width 0.5) (layer F.Cu) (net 20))
 (segment (start 166.4208 71.2724) (end 163.9824 71.2724) (width 0.5) (layer F.Cu) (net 21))
 (segment (start 161.8996 91.0209) (end 158.3055 94.615) (width 0.5) (layer F.Cu) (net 21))
 (segment (start 161.8996 73.3552) (end 161.8996 91.0209) (width 0.5) (layer F.Cu) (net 21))
 (segment (start 163.9824 71.2724) (end 161.8996 73.3552) (width 0.5) (layer F.Cu) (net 21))
 (segment (start 166.4208 73.8124) (end 163.9824 73.8124) (width 0.5) (layer F.Cu) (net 22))
 (segment (start 161.0614 99.695) (end 158.3055 99.695) (width 0.5) (layer F.Cu) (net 22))
 (segment (start 163.4744 97.282) (end 161.0614 99.695) (width 0.5) (layer F.Cu) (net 22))
 (segment (start 163.4744 74.3204) (end 163.4744 97.282) (width 0.5) (layer F.Cu) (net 22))
 (segment (start 163.9824 73.8124) (end 163.4744 74.3204) (width 0.5) (layer F.Cu) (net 22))
 (segment (start 186.9186 53.975) (end 158.3055 53.975) (width 0.5) (layer F.Cu) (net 23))
 (segment (start 189.992 57.0484) (end 186.9186 53.975) (width 0.5) (layer F.Cu) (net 23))
 (segment (start 189.992 82.3468) (end 189.992 57.0484) (width 0.5) (layer F.Cu) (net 23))
 (segment (start 188.1124 84.2264) (end 189.992 82.3468) (width 0.5) (layer F.Cu) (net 23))
 (segment (start 168.1988 84.2264) (end 188.1124 84.2264) (width 0.5) (layer F.Cu) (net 23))
 (segment (start 166.4208 82.4484) (end 168.1988 84.2264) (width 0.5) (layer F.Cu) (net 23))
 (segment (start 166.4208 76.3524) (end 166.4208 82.4484) (width 0.5) (layer F.Cu) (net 23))
 (segment (start 135.382 58.9915) (end 126.4793 58.9915) (width 0.5) (layer F.Cu) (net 30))
 (segment (start 121.92 70.5104) (end 117.2464 70.5104) (width 0.5) (layer F.Cu) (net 30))
 (segment (start 124.8664 67.564) (end 121.92 70.5104) (width 0.5) (layer F.Cu) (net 30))
 (segment (start 124.8664 60.6044) (end 124.8664 67.564) (width 0.5) (layer F.Cu) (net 30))
 (segment (start 126.4793 58.9915) (end 124.8664 60.6044) (width 0.5) (layer F.Cu) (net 30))
 (segment (start 117.2464 73.0504) (end 113.9952 73.0504) (width 0.5) (layer F.Cu) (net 31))
 (segment (start 111.9505 75.0951) (end 111.9505 94.107) (width 0.5) (layer F.Cu) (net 31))
 (segment (start 113.9952 73.0504) (end 111.9505 75.0951) (width 0.5) (layer F.Cu) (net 31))
 (segment (start 139.192 107.8484) (end 139.192 104.3432) (width 0.5) (layer F.Cu) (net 31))
 (segment (start 142.6972 68.8467) (end 135.382 61.5315) (width 0.5) (layer F.Cu) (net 31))
 (segment (start 142.6972 100.838) (end 142.6972 68.8467) (width 0.5) (layer F.Cu) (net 31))
 (segment (start 139.192 104.3432) (end 142.6972 100.838) (width 0.5) (layer F.Cu) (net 31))
 (segment (start 135.382 61.5315) (end 130.7465 61.5315) (width 0.5) (layer F.Cu) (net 31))
 (segment (start 123.19 73.0504) (end 117.2464 73.0504) (width 0.5) (layer F.Cu) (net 31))
 (segment (start 127.508 68.7324) (end 123.19 73.0504) (width 0.5) (layer F.Cu) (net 31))
 (segment (start 127.508 64.77) (end 127.508 68.7324) (width 0.5) (layer F.Cu) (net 31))
 (segment (start 130.7465 61.5315) (end 127.508 64.77) (width 0.5) (layer F.Cu) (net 31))
 (segment (start 135.382 71.6915) (end 130.1369 71.6915) (width 0.5) (layer F.Cu) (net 35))
 (segment (start 123.3424 83.2104) (end 117.2464 83.2104) (width 0.5) (layer F.Cu) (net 35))
 (segment (start 123.3424 78.486) (end 123.3424 83.2104) (width 0.5) (layer F.Cu) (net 35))
 (segment (start 130.1369 71.6915) (end 123.3424 78.486) (width 0.5) (layer F.Cu) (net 35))
 (segment (start 158.3055 97.155) (end 154.2034 97.155) (width 0.5) (layer F.Cu) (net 45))
 (segment (start 147.2184 107.8484) (end 141.732 107.8484) (width 0.5) (layer F.Cu) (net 45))
 (segment (start 149.3012 105.7656) (end 147.2184 107.8484) (width 0.5) (layer F.Cu) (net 45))
 (segment (start 149.3012 102.0572) (end 149.3012 105.7656) (width 0.5) (layer F.Cu) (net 45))
 (segment (start 154.2034 97.155) (end 149.3012 102.0572) (width 0.5) (layer F.Cu) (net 45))
 (segment (start 109.4105 94.107) (end 106.7054 94.107) (width 0.5) (layer F.Cu) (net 60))
 (segment (start 104.521 91.9226) (end 104.521 83.3755) (width 0.5) (layer F.Cu) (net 60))
 (segment (start 106.7054 94.107) (end 104.521 91.9226) (width 0.5) (layer F.Cu) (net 60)))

